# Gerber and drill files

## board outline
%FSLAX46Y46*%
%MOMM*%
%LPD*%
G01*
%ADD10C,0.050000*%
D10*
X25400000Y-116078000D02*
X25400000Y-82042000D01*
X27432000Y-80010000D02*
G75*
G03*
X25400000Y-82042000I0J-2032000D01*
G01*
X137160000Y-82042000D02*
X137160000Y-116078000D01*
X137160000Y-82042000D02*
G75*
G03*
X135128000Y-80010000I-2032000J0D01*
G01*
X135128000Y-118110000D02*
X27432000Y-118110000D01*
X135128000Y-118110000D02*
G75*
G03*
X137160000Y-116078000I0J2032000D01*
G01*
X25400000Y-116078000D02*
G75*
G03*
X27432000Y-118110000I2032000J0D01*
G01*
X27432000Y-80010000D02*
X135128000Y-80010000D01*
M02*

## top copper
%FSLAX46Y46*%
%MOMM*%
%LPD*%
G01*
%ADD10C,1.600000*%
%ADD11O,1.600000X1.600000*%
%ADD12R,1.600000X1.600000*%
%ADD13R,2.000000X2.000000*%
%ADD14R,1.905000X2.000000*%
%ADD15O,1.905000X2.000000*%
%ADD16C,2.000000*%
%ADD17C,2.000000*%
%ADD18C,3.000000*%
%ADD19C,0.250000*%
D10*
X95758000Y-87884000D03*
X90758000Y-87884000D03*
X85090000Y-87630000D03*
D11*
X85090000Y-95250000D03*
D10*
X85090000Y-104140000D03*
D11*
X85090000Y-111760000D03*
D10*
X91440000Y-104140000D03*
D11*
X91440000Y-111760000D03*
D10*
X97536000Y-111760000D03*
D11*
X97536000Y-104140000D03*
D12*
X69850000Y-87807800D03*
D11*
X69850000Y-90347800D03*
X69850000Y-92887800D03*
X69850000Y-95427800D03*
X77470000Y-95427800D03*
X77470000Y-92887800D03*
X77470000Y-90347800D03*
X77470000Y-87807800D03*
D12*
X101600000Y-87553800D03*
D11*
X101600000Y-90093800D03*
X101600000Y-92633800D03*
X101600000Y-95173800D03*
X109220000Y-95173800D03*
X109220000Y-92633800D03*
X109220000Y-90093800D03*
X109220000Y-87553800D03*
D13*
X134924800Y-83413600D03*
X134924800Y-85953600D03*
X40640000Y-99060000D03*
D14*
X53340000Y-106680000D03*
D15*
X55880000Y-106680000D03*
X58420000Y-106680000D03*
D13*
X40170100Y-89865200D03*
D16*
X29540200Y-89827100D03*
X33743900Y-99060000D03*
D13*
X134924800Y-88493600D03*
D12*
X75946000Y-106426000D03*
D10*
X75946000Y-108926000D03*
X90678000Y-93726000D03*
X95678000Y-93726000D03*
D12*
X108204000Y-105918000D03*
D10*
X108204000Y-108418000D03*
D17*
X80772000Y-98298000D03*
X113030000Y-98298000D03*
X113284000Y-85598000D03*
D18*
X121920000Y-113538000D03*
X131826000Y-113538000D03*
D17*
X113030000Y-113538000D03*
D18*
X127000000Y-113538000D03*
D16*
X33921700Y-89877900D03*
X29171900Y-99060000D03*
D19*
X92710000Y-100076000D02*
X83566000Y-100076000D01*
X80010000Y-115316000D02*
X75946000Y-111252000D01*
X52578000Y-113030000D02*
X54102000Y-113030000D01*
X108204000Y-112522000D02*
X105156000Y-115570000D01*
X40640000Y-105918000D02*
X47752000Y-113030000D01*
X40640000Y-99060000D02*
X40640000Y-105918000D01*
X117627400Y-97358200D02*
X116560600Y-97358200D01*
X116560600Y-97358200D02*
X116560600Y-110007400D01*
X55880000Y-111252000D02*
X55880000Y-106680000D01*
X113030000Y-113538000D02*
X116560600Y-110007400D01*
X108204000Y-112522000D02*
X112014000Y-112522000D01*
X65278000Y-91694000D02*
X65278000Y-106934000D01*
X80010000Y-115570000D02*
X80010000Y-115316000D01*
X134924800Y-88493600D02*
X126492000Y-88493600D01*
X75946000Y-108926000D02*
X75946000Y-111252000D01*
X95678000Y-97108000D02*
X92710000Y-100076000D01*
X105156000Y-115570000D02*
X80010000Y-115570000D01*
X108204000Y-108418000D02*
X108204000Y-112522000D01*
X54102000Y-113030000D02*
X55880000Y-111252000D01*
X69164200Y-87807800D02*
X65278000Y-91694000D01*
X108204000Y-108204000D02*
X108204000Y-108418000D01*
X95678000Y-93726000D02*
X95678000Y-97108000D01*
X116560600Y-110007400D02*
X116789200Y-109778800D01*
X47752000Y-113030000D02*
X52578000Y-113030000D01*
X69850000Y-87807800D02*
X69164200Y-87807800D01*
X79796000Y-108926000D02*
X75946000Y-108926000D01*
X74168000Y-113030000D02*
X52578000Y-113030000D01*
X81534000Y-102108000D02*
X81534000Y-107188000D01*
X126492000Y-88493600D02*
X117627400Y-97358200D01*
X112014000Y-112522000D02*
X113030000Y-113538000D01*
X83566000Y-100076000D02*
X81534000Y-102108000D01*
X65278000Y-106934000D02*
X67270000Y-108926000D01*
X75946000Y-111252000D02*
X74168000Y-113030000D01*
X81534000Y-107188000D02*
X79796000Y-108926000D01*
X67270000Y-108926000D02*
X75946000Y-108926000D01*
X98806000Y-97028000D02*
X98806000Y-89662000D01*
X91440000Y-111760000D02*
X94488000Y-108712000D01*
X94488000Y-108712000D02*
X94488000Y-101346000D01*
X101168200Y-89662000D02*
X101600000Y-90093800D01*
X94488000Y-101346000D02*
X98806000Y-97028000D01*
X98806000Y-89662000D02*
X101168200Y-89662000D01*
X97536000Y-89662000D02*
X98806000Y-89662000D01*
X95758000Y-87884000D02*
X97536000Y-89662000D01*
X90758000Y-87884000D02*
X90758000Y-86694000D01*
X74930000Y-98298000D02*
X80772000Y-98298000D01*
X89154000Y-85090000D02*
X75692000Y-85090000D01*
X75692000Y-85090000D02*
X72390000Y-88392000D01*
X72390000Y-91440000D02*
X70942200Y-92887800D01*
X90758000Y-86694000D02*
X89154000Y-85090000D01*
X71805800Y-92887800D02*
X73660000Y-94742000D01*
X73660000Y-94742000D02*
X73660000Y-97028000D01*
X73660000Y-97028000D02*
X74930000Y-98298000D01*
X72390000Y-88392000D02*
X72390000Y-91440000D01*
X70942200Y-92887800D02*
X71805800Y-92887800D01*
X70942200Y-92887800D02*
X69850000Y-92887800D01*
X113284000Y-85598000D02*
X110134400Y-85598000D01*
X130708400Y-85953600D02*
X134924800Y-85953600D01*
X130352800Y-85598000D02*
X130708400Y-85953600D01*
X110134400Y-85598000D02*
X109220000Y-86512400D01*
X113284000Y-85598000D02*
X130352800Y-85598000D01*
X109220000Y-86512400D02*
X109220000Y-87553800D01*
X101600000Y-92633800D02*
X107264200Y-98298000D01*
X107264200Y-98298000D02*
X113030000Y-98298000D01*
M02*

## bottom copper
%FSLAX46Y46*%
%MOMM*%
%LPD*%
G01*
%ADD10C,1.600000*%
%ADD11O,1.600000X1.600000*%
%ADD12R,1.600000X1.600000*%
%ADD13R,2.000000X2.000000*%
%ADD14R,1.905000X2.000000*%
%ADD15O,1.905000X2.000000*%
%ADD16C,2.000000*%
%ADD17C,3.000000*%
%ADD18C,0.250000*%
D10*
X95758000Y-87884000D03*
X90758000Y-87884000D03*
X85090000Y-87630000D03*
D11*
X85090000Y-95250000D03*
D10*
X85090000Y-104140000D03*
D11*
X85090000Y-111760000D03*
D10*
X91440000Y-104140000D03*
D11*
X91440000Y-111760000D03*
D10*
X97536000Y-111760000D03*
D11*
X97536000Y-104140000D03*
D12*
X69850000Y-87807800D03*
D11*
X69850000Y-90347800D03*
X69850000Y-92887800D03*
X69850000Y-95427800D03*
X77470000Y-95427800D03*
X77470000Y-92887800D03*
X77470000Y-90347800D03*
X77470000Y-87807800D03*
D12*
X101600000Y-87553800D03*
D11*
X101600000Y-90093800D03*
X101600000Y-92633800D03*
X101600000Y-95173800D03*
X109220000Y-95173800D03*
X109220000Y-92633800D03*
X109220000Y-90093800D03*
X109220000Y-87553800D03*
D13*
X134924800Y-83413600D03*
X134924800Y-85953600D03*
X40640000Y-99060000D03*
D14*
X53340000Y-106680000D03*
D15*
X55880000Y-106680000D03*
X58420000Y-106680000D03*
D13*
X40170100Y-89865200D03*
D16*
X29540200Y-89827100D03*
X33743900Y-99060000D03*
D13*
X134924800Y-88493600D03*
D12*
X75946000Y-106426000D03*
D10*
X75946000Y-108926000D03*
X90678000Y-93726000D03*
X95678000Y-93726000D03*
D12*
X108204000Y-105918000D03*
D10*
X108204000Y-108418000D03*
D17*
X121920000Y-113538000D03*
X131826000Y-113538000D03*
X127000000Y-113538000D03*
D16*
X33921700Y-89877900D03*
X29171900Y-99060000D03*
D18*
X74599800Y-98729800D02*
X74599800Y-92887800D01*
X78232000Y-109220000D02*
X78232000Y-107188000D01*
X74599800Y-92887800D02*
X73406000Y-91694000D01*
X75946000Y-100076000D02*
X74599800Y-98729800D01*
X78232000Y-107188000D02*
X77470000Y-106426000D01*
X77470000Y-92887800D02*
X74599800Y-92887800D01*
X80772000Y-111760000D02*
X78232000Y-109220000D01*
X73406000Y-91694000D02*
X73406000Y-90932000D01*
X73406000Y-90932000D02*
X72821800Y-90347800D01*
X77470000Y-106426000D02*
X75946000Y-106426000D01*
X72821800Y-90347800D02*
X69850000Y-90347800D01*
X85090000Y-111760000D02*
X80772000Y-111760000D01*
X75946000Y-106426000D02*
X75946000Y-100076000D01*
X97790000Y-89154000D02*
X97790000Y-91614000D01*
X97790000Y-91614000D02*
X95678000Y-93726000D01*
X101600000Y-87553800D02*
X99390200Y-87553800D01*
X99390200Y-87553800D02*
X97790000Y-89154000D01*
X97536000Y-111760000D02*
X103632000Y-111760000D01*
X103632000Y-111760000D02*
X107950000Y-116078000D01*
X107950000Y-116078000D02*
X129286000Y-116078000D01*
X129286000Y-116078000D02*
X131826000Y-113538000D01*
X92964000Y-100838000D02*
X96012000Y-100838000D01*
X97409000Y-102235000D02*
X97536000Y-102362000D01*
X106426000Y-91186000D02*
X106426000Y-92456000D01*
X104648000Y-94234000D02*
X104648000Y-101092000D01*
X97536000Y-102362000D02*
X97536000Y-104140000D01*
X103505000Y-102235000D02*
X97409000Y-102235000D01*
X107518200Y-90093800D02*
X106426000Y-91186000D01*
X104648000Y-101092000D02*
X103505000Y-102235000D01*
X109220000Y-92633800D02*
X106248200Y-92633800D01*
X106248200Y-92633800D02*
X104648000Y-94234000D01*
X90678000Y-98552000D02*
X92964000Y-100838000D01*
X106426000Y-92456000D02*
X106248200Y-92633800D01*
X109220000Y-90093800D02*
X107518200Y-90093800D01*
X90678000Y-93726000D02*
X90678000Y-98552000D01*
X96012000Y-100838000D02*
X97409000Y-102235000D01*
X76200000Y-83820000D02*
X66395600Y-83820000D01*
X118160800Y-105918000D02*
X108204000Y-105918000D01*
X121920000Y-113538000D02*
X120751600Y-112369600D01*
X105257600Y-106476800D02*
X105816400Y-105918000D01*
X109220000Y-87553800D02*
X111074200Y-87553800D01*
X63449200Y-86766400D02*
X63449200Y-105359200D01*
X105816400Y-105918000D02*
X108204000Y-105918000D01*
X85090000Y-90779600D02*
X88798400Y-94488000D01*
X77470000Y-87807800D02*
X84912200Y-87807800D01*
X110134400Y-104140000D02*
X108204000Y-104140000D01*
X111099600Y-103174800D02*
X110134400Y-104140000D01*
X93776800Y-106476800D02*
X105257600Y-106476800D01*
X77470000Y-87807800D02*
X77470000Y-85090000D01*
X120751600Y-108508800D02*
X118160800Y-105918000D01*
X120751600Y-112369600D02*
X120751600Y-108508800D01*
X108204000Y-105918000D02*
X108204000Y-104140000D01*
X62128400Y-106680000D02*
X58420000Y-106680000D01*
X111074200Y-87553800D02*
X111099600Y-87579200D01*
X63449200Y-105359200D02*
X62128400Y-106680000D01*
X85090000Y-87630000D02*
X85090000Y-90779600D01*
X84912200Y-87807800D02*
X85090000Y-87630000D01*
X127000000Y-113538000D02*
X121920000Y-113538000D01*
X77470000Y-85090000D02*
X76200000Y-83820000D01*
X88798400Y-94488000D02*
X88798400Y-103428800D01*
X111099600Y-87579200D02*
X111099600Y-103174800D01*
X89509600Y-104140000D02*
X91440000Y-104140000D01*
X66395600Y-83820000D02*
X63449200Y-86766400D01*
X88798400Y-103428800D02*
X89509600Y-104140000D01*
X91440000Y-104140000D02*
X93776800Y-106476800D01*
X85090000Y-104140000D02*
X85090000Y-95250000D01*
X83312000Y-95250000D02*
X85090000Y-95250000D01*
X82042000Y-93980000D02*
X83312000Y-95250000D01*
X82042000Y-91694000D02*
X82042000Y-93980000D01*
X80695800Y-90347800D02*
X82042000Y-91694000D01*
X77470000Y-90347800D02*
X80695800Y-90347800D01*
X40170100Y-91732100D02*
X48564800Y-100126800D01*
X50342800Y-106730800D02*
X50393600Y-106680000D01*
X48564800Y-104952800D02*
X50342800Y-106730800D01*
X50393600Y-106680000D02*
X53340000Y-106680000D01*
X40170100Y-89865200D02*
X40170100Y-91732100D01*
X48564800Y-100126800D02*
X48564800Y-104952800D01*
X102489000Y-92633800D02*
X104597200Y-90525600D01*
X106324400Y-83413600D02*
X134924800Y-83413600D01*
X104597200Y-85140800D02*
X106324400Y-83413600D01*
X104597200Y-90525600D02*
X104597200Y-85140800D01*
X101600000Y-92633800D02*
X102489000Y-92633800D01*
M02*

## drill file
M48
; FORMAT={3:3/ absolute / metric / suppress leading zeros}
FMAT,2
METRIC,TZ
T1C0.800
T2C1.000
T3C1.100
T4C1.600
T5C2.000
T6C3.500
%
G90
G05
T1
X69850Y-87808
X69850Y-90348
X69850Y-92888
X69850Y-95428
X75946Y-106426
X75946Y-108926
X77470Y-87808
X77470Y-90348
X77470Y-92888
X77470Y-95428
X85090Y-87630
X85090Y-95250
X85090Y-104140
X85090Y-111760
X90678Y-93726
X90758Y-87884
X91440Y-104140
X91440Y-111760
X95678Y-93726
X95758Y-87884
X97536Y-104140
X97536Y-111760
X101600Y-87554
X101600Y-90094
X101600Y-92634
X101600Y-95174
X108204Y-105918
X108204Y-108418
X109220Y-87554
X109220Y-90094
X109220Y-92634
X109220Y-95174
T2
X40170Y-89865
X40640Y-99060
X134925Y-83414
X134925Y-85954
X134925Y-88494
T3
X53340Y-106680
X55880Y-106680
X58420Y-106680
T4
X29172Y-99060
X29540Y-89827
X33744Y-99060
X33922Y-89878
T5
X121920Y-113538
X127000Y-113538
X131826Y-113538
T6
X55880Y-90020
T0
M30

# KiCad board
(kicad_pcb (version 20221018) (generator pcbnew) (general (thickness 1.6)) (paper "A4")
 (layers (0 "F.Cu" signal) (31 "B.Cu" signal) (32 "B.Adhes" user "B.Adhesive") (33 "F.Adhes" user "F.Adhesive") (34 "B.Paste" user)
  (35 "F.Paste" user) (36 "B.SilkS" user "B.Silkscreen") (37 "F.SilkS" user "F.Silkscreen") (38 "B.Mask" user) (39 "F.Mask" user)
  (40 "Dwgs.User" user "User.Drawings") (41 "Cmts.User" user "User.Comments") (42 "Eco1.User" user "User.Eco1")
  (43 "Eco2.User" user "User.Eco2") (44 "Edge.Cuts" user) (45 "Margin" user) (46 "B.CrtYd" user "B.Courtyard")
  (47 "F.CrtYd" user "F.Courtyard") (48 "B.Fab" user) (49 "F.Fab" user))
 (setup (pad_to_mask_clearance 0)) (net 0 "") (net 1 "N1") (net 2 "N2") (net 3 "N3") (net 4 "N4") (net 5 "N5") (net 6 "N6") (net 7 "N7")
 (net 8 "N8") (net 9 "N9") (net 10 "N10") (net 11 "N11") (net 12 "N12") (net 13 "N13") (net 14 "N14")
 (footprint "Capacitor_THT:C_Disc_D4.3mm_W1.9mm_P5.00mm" (layer "F.Cu") (at 95.758 87.884 180)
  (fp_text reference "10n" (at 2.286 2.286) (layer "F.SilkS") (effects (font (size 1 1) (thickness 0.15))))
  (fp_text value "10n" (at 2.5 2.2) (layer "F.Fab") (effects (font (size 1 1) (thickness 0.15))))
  (pad "1" thru_hole circle (at 0 0 180) (size 1.6 1.6) (drill 0.8) (layers "*.Cu" "*.Mask") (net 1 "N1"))
  (pad "2" thru_hole circle (at 5 0 180) (size 1.6 1.6) (drill 0.8) (layers "*.Cu" "*.Mask") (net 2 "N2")))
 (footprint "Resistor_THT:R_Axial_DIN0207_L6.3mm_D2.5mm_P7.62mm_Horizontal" (layer "F.Cu") (at 85.09 87.63 -90)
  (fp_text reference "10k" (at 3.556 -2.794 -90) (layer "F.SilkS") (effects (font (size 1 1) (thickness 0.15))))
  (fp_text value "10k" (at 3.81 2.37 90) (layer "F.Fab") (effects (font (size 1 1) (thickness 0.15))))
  (pad "1" thru_hole circle (at 0 0 270) (size 1.6 1.6) (drill 0.8) (layers "*.Cu" "*.Mask") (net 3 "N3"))
  (pad "2" thru_hole oval (at 7.62 0 270) (size 1.6 1.6) (drill 0.8) (layers "*.Cu" "*.Mask") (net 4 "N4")))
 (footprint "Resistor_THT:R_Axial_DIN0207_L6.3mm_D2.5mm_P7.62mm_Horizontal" (layer "F.Cu") (at 85.09 104.14 -90)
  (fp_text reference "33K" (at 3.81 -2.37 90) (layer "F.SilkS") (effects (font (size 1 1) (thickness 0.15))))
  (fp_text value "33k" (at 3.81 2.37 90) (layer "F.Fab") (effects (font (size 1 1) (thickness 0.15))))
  (pad "1" thru_hole circle (at 0 0 270) (size 1.6 1.6) (drill 0.8) (layers "*.Cu" "*.Mask") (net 4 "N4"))
  (pad "2" thru_hole oval (at 7.62 0 270) (size 1.6 1.6) (drill 0.8) (layers "*.Cu" "*.Mask") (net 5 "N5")))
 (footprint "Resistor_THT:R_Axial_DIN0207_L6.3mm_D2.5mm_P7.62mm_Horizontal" (layer "F.Cu") (at 91.44 104.14 -90)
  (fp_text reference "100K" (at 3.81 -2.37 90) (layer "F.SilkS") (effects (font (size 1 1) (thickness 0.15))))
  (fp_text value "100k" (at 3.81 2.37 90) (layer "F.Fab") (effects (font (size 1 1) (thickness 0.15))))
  (pad "1" thru_hole circle (at 0 0 270) (size 1.6 1.6) (drill 0.8) (layers "*.Cu" "*.Mask") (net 3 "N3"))
  (pad "2" thru_hole oval (at 7.62 0 270) (size 1.6 1.6) (drill 0.8) (layers "*.Cu" "*.Mask") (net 1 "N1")))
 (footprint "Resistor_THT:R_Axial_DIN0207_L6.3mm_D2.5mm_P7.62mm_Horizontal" (layer "F.Cu") (at 97.536 111.76 90)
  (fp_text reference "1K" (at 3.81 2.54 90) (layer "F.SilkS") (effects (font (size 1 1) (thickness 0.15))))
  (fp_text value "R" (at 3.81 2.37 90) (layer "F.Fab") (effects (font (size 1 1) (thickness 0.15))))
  (pad "1" thru_hole circle (at 0 0 90) (size 1.6 1.6) (drill 0.8) (layers "*.Cu" "*.Mask") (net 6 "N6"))
  (pad "2" thru_hole oval (at 7.62 0 90) (size 1.6 1.6) (drill 0.8) (layers "*.Cu" "*.Mask") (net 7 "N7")))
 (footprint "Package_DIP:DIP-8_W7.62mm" (layer "F.Cu") (at 69.85 87.8078)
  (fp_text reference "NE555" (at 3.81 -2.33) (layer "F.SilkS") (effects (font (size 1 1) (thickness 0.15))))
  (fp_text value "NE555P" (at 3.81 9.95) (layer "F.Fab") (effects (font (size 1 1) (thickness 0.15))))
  (pad "1" thru_hole rect (at 0 0) (size 1.6 1.6) (drill 0.8) (layers "*.Cu" "*.Mask") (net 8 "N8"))
  (pad "2" thru_hole oval (at 0 2.54) (size 1.6 1.6) (drill 0.8) (layers "*.Cu" "*.Mask") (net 5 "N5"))
  (pad "3" thru_hole oval (at 0 5.08) (size 1.6 1.6) (drill 0.8) (layers "*.Cu" "*.Mask") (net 2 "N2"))
  (pad "4" thru_hole oval (at 0 7.62) (size 1.6 1.6) (drill 0.8) (layers "*.Cu" "*.Mask") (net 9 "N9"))
  (pad "5" thru_hole oval (at 7.62 7.62) (size 1.6 1.6) (drill 0.8) (layers "*.Cu" "*.Mask") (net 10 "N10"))
  (pad "6" thru_hole oval (at 7.62 5.08) (size 1.6 1.6) (drill 0.8) (layers "*.Cu" "*.Mask") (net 5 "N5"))
  (pad "7" thru_hole oval (at 7.62 2.54) (size 1.6 1.6) (drill 0.8) (layers "*.Cu" "*.Mask") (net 4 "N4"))
  (pad "8" thru_hole oval (at 7.62 0) (size 1.6 1.6) (drill 0.8) (layers "*.Cu" "*.Mask") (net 3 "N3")))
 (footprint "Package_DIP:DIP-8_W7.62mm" (layer "F.Cu") (at 101.6 87.5538)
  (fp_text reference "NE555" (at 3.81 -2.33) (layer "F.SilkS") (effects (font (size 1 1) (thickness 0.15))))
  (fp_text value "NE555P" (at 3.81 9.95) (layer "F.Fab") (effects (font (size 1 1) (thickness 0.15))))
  (pad "1" thru_hole rect (at 0 0) (size 1.6 1.6) (drill 0.8) (layers "*.Cu" "*.Mask") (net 8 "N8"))
  (pad "2" thru_hole oval (at 0 2.54) (size 1.6 1.6) (drill 0.8) (layers "*.Cu" "*.Mask") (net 1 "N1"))
  (pad "3" thru_hole oval (at 0 5.08) (size 1.6 1.6) (drill 0.8) (layers "*.Cu" "*.Mask") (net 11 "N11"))
  (pad "4" thru_hole oval (at 0 7.62) (size 1.6 1.6) (drill 0.8) (layers "*.Cu" "*.Mask") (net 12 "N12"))
  (pad "5" thru_hole oval (at 7.62 7.62) (size 1.6 1.6) (drill 0.8) (layers "*.Cu" "*.Mask") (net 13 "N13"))
  (pad "6" thru_hole oval (at 7.62 5.08) (size 1.6 1.6) (drill 0.8) (layers "*.Cu" "*.Mask") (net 7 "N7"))
  (pad "7" thru_hole oval (at 7.62 2.54) (size 1.6 1.6) (drill 0.8) (layers "*.Cu" "*.Mask") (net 7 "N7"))
  (pad "8" thru_hole oval (at 7.62 0) (size 1.6 1.6) (drill 0.8) (layers "*.Cu" "*.Mask") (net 3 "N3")))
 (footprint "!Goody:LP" (layer "F.Cu") (at 134.9248 83.4136)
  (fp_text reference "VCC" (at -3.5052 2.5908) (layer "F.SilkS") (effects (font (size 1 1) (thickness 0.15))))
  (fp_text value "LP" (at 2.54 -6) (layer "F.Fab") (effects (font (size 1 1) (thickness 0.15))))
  (pad "1" thru_hole rect (at 0 0) (size 2 2) (drill 1) (layers "*.Cu" "*.Mask") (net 11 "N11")))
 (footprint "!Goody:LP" (layer "F.Cu") (at 134.9248 85.9536)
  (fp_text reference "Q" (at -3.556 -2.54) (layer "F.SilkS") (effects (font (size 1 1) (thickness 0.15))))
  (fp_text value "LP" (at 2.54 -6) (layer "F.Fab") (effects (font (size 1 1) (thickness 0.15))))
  (pad "1" thru_hole rect (at 0 0) (size 2 2) (drill 1) (layers "*.Cu" "*.Mask") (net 3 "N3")))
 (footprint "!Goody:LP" (layer "F.Cu") (at 40.64 99.06)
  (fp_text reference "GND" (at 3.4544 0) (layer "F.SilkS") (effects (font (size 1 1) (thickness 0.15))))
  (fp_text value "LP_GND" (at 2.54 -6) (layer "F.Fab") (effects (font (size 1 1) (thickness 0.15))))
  (pad "1" thru_hole rect (at 0 0) (size 2 2) (drill 1) (layers "*.Cu" "*.Mask") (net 8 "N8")))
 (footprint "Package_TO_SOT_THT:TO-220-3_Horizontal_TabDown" (layer "F.Cu") (at 53.34 106.68)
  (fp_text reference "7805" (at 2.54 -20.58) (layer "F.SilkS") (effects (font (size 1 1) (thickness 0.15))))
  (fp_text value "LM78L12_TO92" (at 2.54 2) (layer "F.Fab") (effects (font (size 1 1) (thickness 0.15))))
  (pad "" np_thru_hole oval (at 2.54 -16.66) (size 3.5 3.5) (drill 3.5) (layers "*.Cu" "*.Mask"))
  (pad "1" thru_hole rect (at 0 0) (size 1.905 2) (drill 1.1) (layers "*.Cu" "*.Mask") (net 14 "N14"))
  (pad "2" thru_hole oval (at 2.54 0) (size 1.905 2) (drill 1.1) (layers "*.Cu" "*.Mask") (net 8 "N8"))
  (pad "3" thru_hole oval (at 5.08 0) (size 1.905 2) (drill 1.1) (layers "*.Cu" "*.Mask") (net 3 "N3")))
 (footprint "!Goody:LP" (layer "F.Cu") (at 40.1701 89.8652)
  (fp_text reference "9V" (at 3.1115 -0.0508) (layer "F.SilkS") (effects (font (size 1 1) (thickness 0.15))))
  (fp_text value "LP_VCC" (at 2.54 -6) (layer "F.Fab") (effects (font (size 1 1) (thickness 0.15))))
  (pad "1" thru_hole rect (at 0 0) (size 2 2) (drill 1) (layers "*.Cu" "*.Mask") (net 14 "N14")))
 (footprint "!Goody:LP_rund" (layer "F.Cu") (at 29.5402 89.8271)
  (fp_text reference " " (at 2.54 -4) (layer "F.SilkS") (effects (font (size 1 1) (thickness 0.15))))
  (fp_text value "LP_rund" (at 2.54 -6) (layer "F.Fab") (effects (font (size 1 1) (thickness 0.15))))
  (pad "1" thru_hole circle (at 0 0) (size 2 2) (drill 1.6) (layers "*.Cu" "*.Mask")))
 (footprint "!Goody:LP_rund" (layer "F.Cu") (at 33.7439 99.06)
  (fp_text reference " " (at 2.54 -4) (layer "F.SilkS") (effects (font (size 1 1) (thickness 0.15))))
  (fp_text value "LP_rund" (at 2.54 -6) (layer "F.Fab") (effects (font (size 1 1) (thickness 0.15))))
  (pad "1" thru_hole circle (at 0 0) (size 2 2) (drill 1.6) (layers "*.Cu" "*.Mask")))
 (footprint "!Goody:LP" (layer "F.Cu") (at 134.9248 88.4936)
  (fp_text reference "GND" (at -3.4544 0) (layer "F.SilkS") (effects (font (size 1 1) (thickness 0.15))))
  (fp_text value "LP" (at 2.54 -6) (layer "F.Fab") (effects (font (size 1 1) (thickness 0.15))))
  (pad "1" thru_hole rect (at 0 0) (size 2 2) (drill 1) (layers "*.Cu" "*.Mask") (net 8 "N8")))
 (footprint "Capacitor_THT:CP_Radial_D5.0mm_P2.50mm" (layer "F.Cu") (at 75.946 106.426 -90)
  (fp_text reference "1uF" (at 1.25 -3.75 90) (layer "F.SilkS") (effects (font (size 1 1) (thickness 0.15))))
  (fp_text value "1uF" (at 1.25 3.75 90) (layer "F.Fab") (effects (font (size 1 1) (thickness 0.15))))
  (pad "1" thru_hole rect (at 0 0 270) (size 1.6 1.6) (drill 0.8) (layers "*.Cu" "*.Mask") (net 5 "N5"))
  (pad "2" thru_hole circle (at 2.5 0 270) (size 1.6 1.6) (drill 0.8) (layers "*.Cu" "*.Mask") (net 8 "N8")))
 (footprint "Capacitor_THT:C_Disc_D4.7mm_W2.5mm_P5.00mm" (layer "F.Cu") (at 90.678 93.726)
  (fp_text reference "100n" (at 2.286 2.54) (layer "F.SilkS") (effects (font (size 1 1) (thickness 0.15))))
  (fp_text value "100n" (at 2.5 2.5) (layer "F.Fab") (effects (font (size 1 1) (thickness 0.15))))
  (pad "1" thru_hole circle (at 0 0) (size 1.6 1.6) (drill 0.8) (layers "*.Cu" "*.Mask") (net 7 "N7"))
  (pad "2" thru_hole circle (at 5 0) (size 1.6 1.6) (drill 0.8) (layers "*.Cu" "*.Mask") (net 8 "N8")))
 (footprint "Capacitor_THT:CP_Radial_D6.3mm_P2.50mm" (layer "F.Cu") (at 108.204 105.918 -90)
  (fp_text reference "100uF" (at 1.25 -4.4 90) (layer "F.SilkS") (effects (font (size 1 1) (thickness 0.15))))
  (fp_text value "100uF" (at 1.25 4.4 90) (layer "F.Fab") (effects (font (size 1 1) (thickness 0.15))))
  (pad "1" thru_hole rect (at 0 0 270) (size 1.6 1.6) (drill 0.8) (layers "*.Cu" "*.Mask") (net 3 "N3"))
  (pad "2" thru_hole circle (at 2.5 0 270) (size 1.6 1.6) (drill 0.8) (layers "*.Cu" "*.Mask") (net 8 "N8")))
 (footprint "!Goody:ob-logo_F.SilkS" (layer "F.Cu") (at 38.1 107.188)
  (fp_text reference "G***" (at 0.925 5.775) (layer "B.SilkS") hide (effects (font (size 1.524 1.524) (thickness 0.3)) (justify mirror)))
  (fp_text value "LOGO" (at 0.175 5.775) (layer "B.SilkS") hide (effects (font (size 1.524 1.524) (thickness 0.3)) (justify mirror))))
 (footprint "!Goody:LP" (layer "F.Cu") (at 80.772 98.298)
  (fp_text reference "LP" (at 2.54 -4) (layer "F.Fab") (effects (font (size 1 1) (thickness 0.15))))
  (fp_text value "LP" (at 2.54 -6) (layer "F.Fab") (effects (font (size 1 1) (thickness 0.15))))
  (pad "1" smd circle (at 0 0) (size 2 2) (layers "F.Cu" "F.Paste" "F.Mask") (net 2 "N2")))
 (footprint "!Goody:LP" (layer "F.Cu") (at 113.03 98.298)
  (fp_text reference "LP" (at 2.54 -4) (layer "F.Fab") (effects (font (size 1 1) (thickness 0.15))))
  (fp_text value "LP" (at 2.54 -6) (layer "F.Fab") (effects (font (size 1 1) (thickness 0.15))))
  (pad "1" smd circle (at 0 0) (size 2 2) (layers "F.Cu" "F.Paste" "F.Mask") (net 11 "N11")))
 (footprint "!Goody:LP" (layer "F.Cu") (at 113.284 85.598)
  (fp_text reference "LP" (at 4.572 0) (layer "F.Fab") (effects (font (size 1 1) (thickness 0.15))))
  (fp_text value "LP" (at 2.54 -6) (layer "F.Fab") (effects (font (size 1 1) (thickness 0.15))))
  (pad "1" smd circle (at 0 0) (size 2 2) (layers "F.Cu" "F.Paste" "F.Mask") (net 3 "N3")))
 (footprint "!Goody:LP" (layer "F.Cu") (at 121.92 113.538 90)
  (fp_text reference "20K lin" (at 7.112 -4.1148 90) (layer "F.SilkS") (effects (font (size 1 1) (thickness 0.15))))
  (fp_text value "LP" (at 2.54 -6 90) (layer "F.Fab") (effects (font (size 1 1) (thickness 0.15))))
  (pad "1" thru_hole circle (at 0 0 90) (size 3 3) (drill 2) (layers "*.Cu" "*.Mask") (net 3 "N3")))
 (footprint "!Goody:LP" (layer "F.Cu") (at 131.826 113.538)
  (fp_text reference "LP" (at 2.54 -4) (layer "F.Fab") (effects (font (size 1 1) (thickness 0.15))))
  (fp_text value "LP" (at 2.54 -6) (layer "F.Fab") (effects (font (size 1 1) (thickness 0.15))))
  (pad "1" thru_hole circle (at 0 0) (size 3 3) (drill 2) (layers "*.Cu" "*.Mask") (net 6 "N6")))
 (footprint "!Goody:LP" (layer "F.Cu") (at 113.03 113.538)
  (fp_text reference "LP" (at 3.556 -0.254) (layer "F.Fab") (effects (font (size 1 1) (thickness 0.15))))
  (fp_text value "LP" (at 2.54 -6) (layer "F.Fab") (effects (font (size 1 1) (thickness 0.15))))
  (pad "1" smd circle (at 0 0) (size 2 2) (layers "F.Cu" "F.Paste" "F.Mask") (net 8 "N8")))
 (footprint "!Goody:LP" (layer "F.Cu") (at 127 113.538)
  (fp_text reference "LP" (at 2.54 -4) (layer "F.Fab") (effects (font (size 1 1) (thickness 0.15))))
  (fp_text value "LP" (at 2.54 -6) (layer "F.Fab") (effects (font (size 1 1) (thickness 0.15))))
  (pad "1" thru_hole circle (at 0 0) (size 3 3) (drill 2) (layers "*.Cu" "*.Mask") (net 3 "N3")))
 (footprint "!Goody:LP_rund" (layer "F.Cu") (at 33.9217 89.8779)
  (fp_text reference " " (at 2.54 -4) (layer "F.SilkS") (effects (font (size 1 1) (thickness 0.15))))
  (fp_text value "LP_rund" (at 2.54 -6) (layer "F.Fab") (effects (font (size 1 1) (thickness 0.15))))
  (pad "1" thru_hole circle (at 0 0) (size 2 2) (drill 1.6) (layers "*.Cu" "*.Mask")))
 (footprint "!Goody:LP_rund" (layer "F.Cu") (at 29.1719 99.06)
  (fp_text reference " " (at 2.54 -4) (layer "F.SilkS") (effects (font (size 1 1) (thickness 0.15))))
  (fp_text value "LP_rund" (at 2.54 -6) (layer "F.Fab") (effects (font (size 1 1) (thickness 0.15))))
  (pad "1" thru_hole circle (at 0 0) (size 2 2) (drill 1.6) (layers "*.Cu" "*.Mask")))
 (gr_line (start 25.4 116.078) (end 25.4 82.042) (stroke (width 0.05) (type solid)) (layer "Edge.Cuts"))
 (gr_arc (start 25.4 82.042) (mid 25.995159 80.605159) (end 27.432 80.01) (stroke (width 0.05) (type solid)) (layer "Edge.Cuts"))
 (gr_line (start 137.16 82.042) (end 137.16 116.078) (stroke (width 0.05) (type solid)) (layer "Edge.Cuts"))
 (gr_arc (start 135.128 80.01) (mid 136.564841 80.605159) (end 137.16 82.042) (stroke (width 0.05) (type solid)) (layer "Edge.Cuts"))
 (gr_line (start 135.128 118.11) (end 27.432 118.11) (stroke (width 0.05) (type solid)) (layer "Edge.Cuts"))
 (gr_arc (start 137.16 116.078) (mid 136.564841 117.514841) (end 135.128 118.11) (stroke (width 0.05) (type solid)) (layer "Edge.Cuts"))
 (gr_arc (start 27.432 118.11) (mid 25.995159 117.514841) (end 25.4 116.078) (stroke (width 0.05) (type solid)) (layer "Edge.Cuts"))
 (gr_line (start 27.432 80.01) (end 135.128 80.01) (stroke (width 0.05) (type solid)) (layer "Edge.Cuts"))
 (segment (start 74.5998 98.7298) (end 74.5998 92.8878) (width 0.25) (layer "B.Cu") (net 5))
 (segment (start 78.232 109.22) (end 78.232 107.188) (width 0.25) (layer "B.Cu") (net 5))
 (segment (start 74.5998 92.8878) (end 73.406 91.694) (width 0.25) (layer "B.Cu") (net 5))
 (segment (start 75.946 100.076) (end 74.5998 98.7298) (width 0.25) (layer "B.Cu") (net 5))
 (segment (start 78.232 107.188) (end 77.47 106.426) (width 0.25) (layer "B.Cu") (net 5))
 (segment (start 77.47 92.8878) (end 74.5998 92.8878) (width 0.25) (layer "B.Cu") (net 5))
 (segment (start 80.772 111.76) (end 78.232 109.22) (width 0.25) (layer "B.Cu") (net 5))
 (segment (start 73.406 91.694) (end 73.406 90.932) (width 0.25) (layer "B.Cu") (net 5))
 (segment (start 73.406 90.932) (end 72.8218 90.3478) (width 0.25) (layer "B.Cu") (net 5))
 (segment (start 77.47 106.426) (end 75.946 106.426) (width 0.25) (layer "B.Cu") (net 5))
 (segment (start 72.8218 90.3478) (end 69.85 90.3478) (width 0.25) (layer "B.Cu") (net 5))
 (segment (start 85.09 111.76) (end 80.772 111.76) (width 0.25) (layer "B.Cu") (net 5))
 (segment (start 75.946 106.426) (end 75.946 100.076) (width 0.25) (layer "B.Cu") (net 5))
 (segment (start 92.71 100.076) (end 83.566 100.076) (width 0.25) (layer "F.Cu") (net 8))
 (segment (start 80.01 115.316) (end 75.946 111.252) (width 0.25) (layer "F.Cu") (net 8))
 (segment (start 52.578 113.03) (end 54.102 113.03) (width 0.25) (layer "F.Cu") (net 8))
 (segment (start 108.204 112.522) (end 105.156 115.57) (width 0.25) (layer "F.Cu") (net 8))
 (segment (start 40.64 105.918) (end 47.752 113.03) (width 0.25) (layer "F.Cu") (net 8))
 (segment (start 40.64 99.06) (end 40.64 105.918) (width 0.25) (layer "F.Cu") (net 8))
 (segment (start 117.6274 97.3582) (end 116.5606 97.3582) (width 0.25) (layer "F.Cu") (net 8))
 (segment (start 116.5606 97.3582) (end 116.5606 110.0074) (width 0.25) (layer "F.Cu") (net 8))
 (segment (start 55.88 111.252) (end 55.88 106.68) (width 0.25) (layer "F.Cu") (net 8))
 (segment (start 113.03 113.538) (end 116.5606 110.0074) (width 0.25) (layer "F.Cu") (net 8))
 (segment (start 108.204 112.522) (end 112.014 112.522) (width 0.25) (layer "F.Cu") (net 8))
 (segment (start 65.278 91.694) (end 65.278 106.934) (width 0.25) (layer "F.Cu") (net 8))
 (segment (start 80.01 115.57) (end 80.01 115.316) (width 0.25) (layer "F.Cu") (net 8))
 (segment (start 134.9248 88.4936) (end 126.492 88.4936) (width 0.25) (layer "F.Cu") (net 8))
 (segment (start 75.946 108.926) (end 75.946 111.252) (width 0.25) (layer "F.Cu") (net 8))
 (segment (start 95.678 97.108) (end 92.71 100.076) (width 0.25) (layer "F.Cu") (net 8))
 (segment (start 105.156 115.57) (end 80.01 115.57) (width 0.25) (layer "F.Cu") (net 8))
 (segment (start 108.204 108.418) (end 108.204 112.522) (width 0.25) (layer "F.Cu") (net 8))
 (segment (start 54.102 113.03) (end 55.88 111.252) (width 0.25) (layer "F.Cu") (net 8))
 (segment (start 69.1642 87.8078) (end 65.278 91.694) (width 0.25) (layer "F.Cu") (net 8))
 (segment (start 108.204 108.204) (end 108.204 108.418) (width 0.25) (layer "F.Cu") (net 8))
 (segment (start 95.678 93.726) (end 95.678 97.108) (width 0.25) (layer "F.Cu") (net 8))
 (segment (start 116.5606 110.0074) (end 116.7892 109.7788) (width 0.25) (layer "F.Cu") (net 8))
 (segment (start 47.752 113.03) (end 52.578 113.03) (width 0.25) (layer "F.Cu") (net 8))
 (segment (start 69.85 87.8078) (end 69.1642 87.8078) (width 0.25) (layer "F.Cu") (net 8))
 (segment (start 79.796 108.926) (end 75.946 108.926) (width 0.25) (layer "F.Cu") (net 8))
 (segment (start 74.168 113.03) (end 52.578 113.03) (width 0.25) (layer "F.Cu") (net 8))
 (segment (start 81.534 102.108) (end 81.534 107.188) (width 0.25) (layer "F.Cu") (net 8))
 (segment (start 126.492 88.4936) (end 117.6274 97.3582) (width 0.25) (layer "F.Cu") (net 8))
 (segment (start 112.014 112.522) (end 113.03 113.538) (width 0.25) (layer "F.Cu") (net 8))
 (segment (start 83.566 100.076) (end 81.534 102.108) (width 0.25) (layer "F.Cu") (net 8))
 (segment (start 65.278 106.934) (end 67.27 108.926) (width 0.25) (layer "F.Cu") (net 8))
 (segment (start 75.946 111.252) (end 74.168 113.03) (width 0.25) (layer "F.Cu") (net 8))
 (segment (start 81.534 107.188) (end 79.796 108.926) (width 0.25) (layer "F.Cu") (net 8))
 (segment (start 67.27 108.926) (end 75.946 108.926) (width 0.25) (layer "F.Cu") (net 8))
 (segment (start 97.79 89.154) (end 97.79 91.614) (width 0.25) (layer "B.Cu") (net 8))
 (segment (start 97.79 91.614) (end 95.678 93.726) (width 0.25) (layer "B.Cu") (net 8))
 (segment (start 101.6 87.5538) (end 99.3902 87.5538) (width 0.25) (layer "B.Cu") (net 8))
 (segment (start 99.3902 87.5538) (end 97.79 89.154) (width 0.25) (layer "B.Cu") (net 8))
 (segment (start 98.806 97.028) (end 98.806 89.662) (width 0.25) (layer "F.Cu") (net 1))
 (segment (start 91.44 111.76) (end 94.488 108.712) (width 0.25) (layer "F.Cu") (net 1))
 (segment (start 94.488 108.712) (end 94.488 101.346) (width 0.25) (layer "F.Cu") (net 1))
 (segment (start 101.1682 89.662) (end 101.6 90.0938) (width 0.25) (layer "F.Cu") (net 1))
 (segment (start 94.488 101.346) (end 98.806 97.028) (width 0.25) (layer "F.Cu") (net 1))
 (segment (start 98.806 89.662) (end 101.1682 89.662) (width 0.25) (layer "F.Cu") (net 1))
 (segment (start 97.536 89.662) (end 98.806 89.662) (width 0.25) (layer "F.Cu") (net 1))
 (segment (start 95.758 87.884) (end 97.536 89.662) (width 0.25) (layer "F.Cu") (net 1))
 (segment (start 90.758 87.884) (end 90.758 86.694) (width 0.25) (layer "F.Cu") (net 2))
 (segment (start 74.93 98.298) (end 80.772 98.298) (width 0.25) (layer "F.Cu") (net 2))
 (segment (start 89.154 85.09) (end 75.692 85.09) (width 0.25) (layer "F.Cu") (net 2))
 (segment (start 75.692 85.09) (end 72.39 88.392) (width 0.25) (layer "F.Cu") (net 2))
 (segment (start 72.39 91.44) (end 70.9422 92.8878) (width 0.25) (layer "F.Cu") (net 2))
 (segment (start 90.758 86.694) (end 89.154 85.09) (width 0.25) (layer "F.Cu") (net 2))
 (segment (start 71.8058 92.8878) (end 73.66 94.742) (width 0.25) (layer "F.Cu") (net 2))
 (segment (start 73.66 94.742) (end 73.66 97.028) (width 0.25) (layer "F.Cu") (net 2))
 (segment (start 73.66 97.028) (end 74.93 98.298) (width 0.25) (layer "F.Cu") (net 2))
 (segment (start 72.39 88.392) (end 72.39 91.44) (width 0.25) (layer "F.Cu") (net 2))
 (segment (start 70.9422 92.8878) (end 71.8058 92.8878) (width 0.25) (layer "F.Cu") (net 2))
 (segment (start 70.9422 92.8878) (end 69.85 92.8878) (width 0.25) (layer "F.Cu") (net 2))
 (segment (start 97.536 111.76) (end 103.632 111.76) (width 0.25) (layer "B.Cu") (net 6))
 (segment (start 103.632 111.76) (end 107.95 116.078) (width 0.25) (layer "B.Cu") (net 6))
 (segment (start 107.95 116.078) (end 129.286 116.078) (width 0.25) (layer "B.Cu") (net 6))
 (segment (start 129.286 116.078) (end 131.826 113.538) (width 0.25) (layer "B.Cu") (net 6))
 (segment (start 92.964 100.838) (end 96.012 100.838) (width 0.25) (layer "B.Cu") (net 7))
 (segment (start 97.409 102.235) (end 97.536 102.362) (width 0.25) (layer "B.Cu") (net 7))
 (segment (start 106.426 91.186) (end 106.426 92.456) (width 0.25) (layer "B.Cu") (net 7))
 (segment (start 104.648 94.234) (end 104.648 101.092) (width 0.25) (layer "B.Cu") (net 7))
 (segment (start 97.536 102.362) (end 97.536 104.14) (width 0.25) (layer "B.Cu") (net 7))
 (segment (start 103.505 102.235) (end 97.409 102.235) (width 0.25) (layer "B.Cu") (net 7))
 (segment (start 107.5182 90.0938) (end 106.426 91.186) (width 0.25) (layer "B.Cu") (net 7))
 (segment (start 104.648 101.092) (end 103.505 102.235) (width 0.25) (layer "B.Cu") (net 7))
 (segment (start 109.22 92.6338) (end 106.2482 92.6338) (width 0.25) (layer "B.Cu") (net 7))
 (segment (start 106.2482 92.6338) (end 104.648 94.234) (width 0.25) (layer "B.Cu") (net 7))
 (segment (start 90.678 98.552) (end 92.964 100.838) (width 0.25) (layer "B.Cu") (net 7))
 (segment (start 106.426 92.456) (end 106.2482 92.6338) (width 0.25) (layer "B.Cu") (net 7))
 (segment (start 109.22 90.0938) (end 107.5182 90.0938) (width 0.25) (layer "B.Cu") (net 7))
 (segment (start 90.678 93.726) (end 90.678 98.552) (width 0.25) (layer "B.Cu") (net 7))
 (segment (start 96.012 100.838) (end 97.409 102.235) (width 0.25) (layer "B.Cu") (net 7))
 (segment (start 113.284 85.598) (end 110.1344 85.598) (width 0.25) (layer "F.Cu") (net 3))
 (segment (start 130.7084 85.9536) (end 134.9248 85.9536) (width 0.25) (layer "F.Cu") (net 3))
 (segment (start 130.3528 85.598) (end 130.7084 85.9536) (width 0.25) (layer "F.Cu") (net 3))
 (segment (start 110.1344 85.598) (end 109.22 86.5124) (width 0.25) (layer "F.Cu") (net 3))
 (segment (start 113.284 85.598) (end 130.3528 85.598) (width 0.25) (layer "F.Cu") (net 3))
 (segment (start 109.22 86.5124) (end 109.22 87.5538) (width 0.25) (layer "F.Cu") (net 3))
 (segment (start 76.2 83.82) (end 66.3956 83.82) (width 0.25) (layer "B.Cu") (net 3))
 (segment (start 118.1608 105.918) (end 108.204 105.918) (width 0.25) (layer "B.Cu") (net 3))
 (segment (start 121.92 113.538) (end 120.7516 112.3696) (width 0.25) (layer "B.Cu") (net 3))
 (segment (start 105.2576 106.4768) (end 105.8164 105.918) (width 0.25) (layer "B.Cu") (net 3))
 (segment (start 109.22 87.5538) (end 111.0742 87.5538) (width 0.25) (layer "B.Cu") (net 3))
 (segment (start 63.4492 86.7664) (end 63.4492 105.3592) (width 0.25) (layer "B.Cu") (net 3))
 (segment (start 105.8164 105.918) (end 108.204 105.918) (width 0.25) (layer "B.Cu") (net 3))
 (segment (start 85.09 90.7796) (end 88.7984 94.488) (width 0.25) (layer "B.Cu") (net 3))
 (segment (start 77.47 87.8078) (end 84.9122 87.8078) (width 0.25) (layer "B.Cu") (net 3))
 (segment (start 110.1344 104.14) (end 108.204 104.14) (width 0.25) (layer "B.Cu") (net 3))
 (segment (start 111.0996 103.1748) (end 110.1344 104.14) (width 0.25) (layer "B.Cu") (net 3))
 (segment (start 93.7768 106.4768) (end 105.2576 106.4768) (width 0.25) (layer "B.Cu") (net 3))
 (segment (start 77.47 87.8078) (end 77.47 85.09) (width 0.25) (layer "B.Cu") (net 3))
 (segment (start 120.7516 108.5088) (end 118.1608 105.918) (width 0.25) (layer "B.Cu") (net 3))
 (segment (start 120.7516 112.3696) (end 120.7516 108.5088) (width 0.25) (layer "B.Cu") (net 3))
 (segment (start 108.204 105.918) (end 108.204 104.14) (width 0.25) (layer "B.Cu") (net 3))
 (segment (start 62.1284 106.68) (end 58.42 106.68) (width 0.25) (layer "B.Cu") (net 3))
 (segment (start 111.0742 87.5538) (end 111.0996 87.5792) (width 0.25) (layer "B.Cu") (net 3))
 (segment (start 63.4492 105.3592) (end 62.1284 106.68) (width 0.25) (layer "B.Cu") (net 3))
 (segment (start 85.09 87.63) (end 85.09 90.7796) (width 0.25) (layer "B.Cu") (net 3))
 (segment (start 84.9122 87.8078) (end 85.09 87.63) (width 0.25) (layer "B.Cu") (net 3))
 (segment (start 127 113.538) (end 121.92 113.538) (width 0.25) (layer "B.Cu") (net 3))
 (segment (start 77.47 85.09) (end 76.2 83.82) (width 0.25) (layer "B.Cu") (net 3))
 (segment (start 88.7984 94.488) (end 88.7984 103.4288) (width 0.25) (layer "B.Cu") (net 3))
 (segment (start 111.0996 87.5792) (end 111.0996 103.1748) (width 0.25) (layer "B.Cu") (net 3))
 (segment (start 89.5096 104.14) (end 91.44 104.14) (width 0.25) (layer "B.Cu") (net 3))
 (segment (start 66.3956 83.82) (end 63.4492 86.7664) (width 0.25) (layer "B.Cu") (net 3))
 (segment (start 88.7984 103.4288) (end 89.5096 104.14) (width 0.25) (layer "B.Cu") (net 3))
 (segment (start 91.44 104.14) (end 93.7768 106.4768) (width 0.25) (layer "B.Cu") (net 3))
 (segment (start 85.09 104.14) (end 85.09 95.25) (width 0.25) (layer "B.Cu") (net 4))
 (segment (start 83.312 95.25) (end 85.09 95.25) (width 0.25) (layer "B.Cu") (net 4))
 (segment (start 82.042 93.98) (end 83.312 95.25) (width 0.25) (layer "B.Cu") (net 4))
 (segment (start 82.042 91.694) (end 82.042 93.98) (width 0.25) (layer "B.Cu") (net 4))
 (segment (start 80.6958 90.3478) (end 82.042 91.694) (width 0.25) (layer "B.Cu") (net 4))
 (segment (start 77.47 90.3478) (end 80.6958 90.3478) (width 0.25) (layer "B.Cu") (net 4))
 (segment (start 40.1701 91.7321) (end 48.5648 100.1268) (width 0.25) (layer "B.Cu") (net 14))
 (segment (start 50.3428 106.7308) (end 50.3936 106.68) (width 0.25) (layer "B.Cu") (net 14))
 (segment (start 48.5648 104.9528) (end 50.3428 106.7308) (width 0.25) (layer "B.Cu") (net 14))
 (segment (start 50.3936 106.68) (end 53.34 106.68) (width 0.25) (layer "B.Cu") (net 14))
 (segment (start 40.1701 89.8652) (end 40.1701 91.7321) (width 0.25) (layer "B.Cu") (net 14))
 (segment (start 48.5648 100.1268) (end 48.5648 104.9528) (width 0.25) (layer "B.Cu") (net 14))
 (segment (start 101.6 92.6338) (end 107.2642 98.298) (width 0.25) (layer "F.Cu") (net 11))
 (segment (start 107.2642 98.298) (end 113.03 98.298) (width 0.25) (layer "F.Cu") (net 11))
 (segment (start 102.489 92.6338) (end 104.5972 90.5256) (width 0.25) (layer "B.Cu") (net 11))
 (segment (start 106.3244 83.4136) (end 134.9248 83.4136) (width 0.25) (layer "B.Cu") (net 11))
 (segment (start 104.5972 85.1408) (end 106.3244 83.4136) (width 0.25) (layer "B.Cu") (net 11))
 (segment (start 104.5972 90.5256) (end 104.5972 85.1408) (width 0.25) (layer "B.Cu") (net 11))
 (segment (start 101.6 92.6338) (end 102.489 92.6338) (width 0.25) (layer "B.Cu") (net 11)))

